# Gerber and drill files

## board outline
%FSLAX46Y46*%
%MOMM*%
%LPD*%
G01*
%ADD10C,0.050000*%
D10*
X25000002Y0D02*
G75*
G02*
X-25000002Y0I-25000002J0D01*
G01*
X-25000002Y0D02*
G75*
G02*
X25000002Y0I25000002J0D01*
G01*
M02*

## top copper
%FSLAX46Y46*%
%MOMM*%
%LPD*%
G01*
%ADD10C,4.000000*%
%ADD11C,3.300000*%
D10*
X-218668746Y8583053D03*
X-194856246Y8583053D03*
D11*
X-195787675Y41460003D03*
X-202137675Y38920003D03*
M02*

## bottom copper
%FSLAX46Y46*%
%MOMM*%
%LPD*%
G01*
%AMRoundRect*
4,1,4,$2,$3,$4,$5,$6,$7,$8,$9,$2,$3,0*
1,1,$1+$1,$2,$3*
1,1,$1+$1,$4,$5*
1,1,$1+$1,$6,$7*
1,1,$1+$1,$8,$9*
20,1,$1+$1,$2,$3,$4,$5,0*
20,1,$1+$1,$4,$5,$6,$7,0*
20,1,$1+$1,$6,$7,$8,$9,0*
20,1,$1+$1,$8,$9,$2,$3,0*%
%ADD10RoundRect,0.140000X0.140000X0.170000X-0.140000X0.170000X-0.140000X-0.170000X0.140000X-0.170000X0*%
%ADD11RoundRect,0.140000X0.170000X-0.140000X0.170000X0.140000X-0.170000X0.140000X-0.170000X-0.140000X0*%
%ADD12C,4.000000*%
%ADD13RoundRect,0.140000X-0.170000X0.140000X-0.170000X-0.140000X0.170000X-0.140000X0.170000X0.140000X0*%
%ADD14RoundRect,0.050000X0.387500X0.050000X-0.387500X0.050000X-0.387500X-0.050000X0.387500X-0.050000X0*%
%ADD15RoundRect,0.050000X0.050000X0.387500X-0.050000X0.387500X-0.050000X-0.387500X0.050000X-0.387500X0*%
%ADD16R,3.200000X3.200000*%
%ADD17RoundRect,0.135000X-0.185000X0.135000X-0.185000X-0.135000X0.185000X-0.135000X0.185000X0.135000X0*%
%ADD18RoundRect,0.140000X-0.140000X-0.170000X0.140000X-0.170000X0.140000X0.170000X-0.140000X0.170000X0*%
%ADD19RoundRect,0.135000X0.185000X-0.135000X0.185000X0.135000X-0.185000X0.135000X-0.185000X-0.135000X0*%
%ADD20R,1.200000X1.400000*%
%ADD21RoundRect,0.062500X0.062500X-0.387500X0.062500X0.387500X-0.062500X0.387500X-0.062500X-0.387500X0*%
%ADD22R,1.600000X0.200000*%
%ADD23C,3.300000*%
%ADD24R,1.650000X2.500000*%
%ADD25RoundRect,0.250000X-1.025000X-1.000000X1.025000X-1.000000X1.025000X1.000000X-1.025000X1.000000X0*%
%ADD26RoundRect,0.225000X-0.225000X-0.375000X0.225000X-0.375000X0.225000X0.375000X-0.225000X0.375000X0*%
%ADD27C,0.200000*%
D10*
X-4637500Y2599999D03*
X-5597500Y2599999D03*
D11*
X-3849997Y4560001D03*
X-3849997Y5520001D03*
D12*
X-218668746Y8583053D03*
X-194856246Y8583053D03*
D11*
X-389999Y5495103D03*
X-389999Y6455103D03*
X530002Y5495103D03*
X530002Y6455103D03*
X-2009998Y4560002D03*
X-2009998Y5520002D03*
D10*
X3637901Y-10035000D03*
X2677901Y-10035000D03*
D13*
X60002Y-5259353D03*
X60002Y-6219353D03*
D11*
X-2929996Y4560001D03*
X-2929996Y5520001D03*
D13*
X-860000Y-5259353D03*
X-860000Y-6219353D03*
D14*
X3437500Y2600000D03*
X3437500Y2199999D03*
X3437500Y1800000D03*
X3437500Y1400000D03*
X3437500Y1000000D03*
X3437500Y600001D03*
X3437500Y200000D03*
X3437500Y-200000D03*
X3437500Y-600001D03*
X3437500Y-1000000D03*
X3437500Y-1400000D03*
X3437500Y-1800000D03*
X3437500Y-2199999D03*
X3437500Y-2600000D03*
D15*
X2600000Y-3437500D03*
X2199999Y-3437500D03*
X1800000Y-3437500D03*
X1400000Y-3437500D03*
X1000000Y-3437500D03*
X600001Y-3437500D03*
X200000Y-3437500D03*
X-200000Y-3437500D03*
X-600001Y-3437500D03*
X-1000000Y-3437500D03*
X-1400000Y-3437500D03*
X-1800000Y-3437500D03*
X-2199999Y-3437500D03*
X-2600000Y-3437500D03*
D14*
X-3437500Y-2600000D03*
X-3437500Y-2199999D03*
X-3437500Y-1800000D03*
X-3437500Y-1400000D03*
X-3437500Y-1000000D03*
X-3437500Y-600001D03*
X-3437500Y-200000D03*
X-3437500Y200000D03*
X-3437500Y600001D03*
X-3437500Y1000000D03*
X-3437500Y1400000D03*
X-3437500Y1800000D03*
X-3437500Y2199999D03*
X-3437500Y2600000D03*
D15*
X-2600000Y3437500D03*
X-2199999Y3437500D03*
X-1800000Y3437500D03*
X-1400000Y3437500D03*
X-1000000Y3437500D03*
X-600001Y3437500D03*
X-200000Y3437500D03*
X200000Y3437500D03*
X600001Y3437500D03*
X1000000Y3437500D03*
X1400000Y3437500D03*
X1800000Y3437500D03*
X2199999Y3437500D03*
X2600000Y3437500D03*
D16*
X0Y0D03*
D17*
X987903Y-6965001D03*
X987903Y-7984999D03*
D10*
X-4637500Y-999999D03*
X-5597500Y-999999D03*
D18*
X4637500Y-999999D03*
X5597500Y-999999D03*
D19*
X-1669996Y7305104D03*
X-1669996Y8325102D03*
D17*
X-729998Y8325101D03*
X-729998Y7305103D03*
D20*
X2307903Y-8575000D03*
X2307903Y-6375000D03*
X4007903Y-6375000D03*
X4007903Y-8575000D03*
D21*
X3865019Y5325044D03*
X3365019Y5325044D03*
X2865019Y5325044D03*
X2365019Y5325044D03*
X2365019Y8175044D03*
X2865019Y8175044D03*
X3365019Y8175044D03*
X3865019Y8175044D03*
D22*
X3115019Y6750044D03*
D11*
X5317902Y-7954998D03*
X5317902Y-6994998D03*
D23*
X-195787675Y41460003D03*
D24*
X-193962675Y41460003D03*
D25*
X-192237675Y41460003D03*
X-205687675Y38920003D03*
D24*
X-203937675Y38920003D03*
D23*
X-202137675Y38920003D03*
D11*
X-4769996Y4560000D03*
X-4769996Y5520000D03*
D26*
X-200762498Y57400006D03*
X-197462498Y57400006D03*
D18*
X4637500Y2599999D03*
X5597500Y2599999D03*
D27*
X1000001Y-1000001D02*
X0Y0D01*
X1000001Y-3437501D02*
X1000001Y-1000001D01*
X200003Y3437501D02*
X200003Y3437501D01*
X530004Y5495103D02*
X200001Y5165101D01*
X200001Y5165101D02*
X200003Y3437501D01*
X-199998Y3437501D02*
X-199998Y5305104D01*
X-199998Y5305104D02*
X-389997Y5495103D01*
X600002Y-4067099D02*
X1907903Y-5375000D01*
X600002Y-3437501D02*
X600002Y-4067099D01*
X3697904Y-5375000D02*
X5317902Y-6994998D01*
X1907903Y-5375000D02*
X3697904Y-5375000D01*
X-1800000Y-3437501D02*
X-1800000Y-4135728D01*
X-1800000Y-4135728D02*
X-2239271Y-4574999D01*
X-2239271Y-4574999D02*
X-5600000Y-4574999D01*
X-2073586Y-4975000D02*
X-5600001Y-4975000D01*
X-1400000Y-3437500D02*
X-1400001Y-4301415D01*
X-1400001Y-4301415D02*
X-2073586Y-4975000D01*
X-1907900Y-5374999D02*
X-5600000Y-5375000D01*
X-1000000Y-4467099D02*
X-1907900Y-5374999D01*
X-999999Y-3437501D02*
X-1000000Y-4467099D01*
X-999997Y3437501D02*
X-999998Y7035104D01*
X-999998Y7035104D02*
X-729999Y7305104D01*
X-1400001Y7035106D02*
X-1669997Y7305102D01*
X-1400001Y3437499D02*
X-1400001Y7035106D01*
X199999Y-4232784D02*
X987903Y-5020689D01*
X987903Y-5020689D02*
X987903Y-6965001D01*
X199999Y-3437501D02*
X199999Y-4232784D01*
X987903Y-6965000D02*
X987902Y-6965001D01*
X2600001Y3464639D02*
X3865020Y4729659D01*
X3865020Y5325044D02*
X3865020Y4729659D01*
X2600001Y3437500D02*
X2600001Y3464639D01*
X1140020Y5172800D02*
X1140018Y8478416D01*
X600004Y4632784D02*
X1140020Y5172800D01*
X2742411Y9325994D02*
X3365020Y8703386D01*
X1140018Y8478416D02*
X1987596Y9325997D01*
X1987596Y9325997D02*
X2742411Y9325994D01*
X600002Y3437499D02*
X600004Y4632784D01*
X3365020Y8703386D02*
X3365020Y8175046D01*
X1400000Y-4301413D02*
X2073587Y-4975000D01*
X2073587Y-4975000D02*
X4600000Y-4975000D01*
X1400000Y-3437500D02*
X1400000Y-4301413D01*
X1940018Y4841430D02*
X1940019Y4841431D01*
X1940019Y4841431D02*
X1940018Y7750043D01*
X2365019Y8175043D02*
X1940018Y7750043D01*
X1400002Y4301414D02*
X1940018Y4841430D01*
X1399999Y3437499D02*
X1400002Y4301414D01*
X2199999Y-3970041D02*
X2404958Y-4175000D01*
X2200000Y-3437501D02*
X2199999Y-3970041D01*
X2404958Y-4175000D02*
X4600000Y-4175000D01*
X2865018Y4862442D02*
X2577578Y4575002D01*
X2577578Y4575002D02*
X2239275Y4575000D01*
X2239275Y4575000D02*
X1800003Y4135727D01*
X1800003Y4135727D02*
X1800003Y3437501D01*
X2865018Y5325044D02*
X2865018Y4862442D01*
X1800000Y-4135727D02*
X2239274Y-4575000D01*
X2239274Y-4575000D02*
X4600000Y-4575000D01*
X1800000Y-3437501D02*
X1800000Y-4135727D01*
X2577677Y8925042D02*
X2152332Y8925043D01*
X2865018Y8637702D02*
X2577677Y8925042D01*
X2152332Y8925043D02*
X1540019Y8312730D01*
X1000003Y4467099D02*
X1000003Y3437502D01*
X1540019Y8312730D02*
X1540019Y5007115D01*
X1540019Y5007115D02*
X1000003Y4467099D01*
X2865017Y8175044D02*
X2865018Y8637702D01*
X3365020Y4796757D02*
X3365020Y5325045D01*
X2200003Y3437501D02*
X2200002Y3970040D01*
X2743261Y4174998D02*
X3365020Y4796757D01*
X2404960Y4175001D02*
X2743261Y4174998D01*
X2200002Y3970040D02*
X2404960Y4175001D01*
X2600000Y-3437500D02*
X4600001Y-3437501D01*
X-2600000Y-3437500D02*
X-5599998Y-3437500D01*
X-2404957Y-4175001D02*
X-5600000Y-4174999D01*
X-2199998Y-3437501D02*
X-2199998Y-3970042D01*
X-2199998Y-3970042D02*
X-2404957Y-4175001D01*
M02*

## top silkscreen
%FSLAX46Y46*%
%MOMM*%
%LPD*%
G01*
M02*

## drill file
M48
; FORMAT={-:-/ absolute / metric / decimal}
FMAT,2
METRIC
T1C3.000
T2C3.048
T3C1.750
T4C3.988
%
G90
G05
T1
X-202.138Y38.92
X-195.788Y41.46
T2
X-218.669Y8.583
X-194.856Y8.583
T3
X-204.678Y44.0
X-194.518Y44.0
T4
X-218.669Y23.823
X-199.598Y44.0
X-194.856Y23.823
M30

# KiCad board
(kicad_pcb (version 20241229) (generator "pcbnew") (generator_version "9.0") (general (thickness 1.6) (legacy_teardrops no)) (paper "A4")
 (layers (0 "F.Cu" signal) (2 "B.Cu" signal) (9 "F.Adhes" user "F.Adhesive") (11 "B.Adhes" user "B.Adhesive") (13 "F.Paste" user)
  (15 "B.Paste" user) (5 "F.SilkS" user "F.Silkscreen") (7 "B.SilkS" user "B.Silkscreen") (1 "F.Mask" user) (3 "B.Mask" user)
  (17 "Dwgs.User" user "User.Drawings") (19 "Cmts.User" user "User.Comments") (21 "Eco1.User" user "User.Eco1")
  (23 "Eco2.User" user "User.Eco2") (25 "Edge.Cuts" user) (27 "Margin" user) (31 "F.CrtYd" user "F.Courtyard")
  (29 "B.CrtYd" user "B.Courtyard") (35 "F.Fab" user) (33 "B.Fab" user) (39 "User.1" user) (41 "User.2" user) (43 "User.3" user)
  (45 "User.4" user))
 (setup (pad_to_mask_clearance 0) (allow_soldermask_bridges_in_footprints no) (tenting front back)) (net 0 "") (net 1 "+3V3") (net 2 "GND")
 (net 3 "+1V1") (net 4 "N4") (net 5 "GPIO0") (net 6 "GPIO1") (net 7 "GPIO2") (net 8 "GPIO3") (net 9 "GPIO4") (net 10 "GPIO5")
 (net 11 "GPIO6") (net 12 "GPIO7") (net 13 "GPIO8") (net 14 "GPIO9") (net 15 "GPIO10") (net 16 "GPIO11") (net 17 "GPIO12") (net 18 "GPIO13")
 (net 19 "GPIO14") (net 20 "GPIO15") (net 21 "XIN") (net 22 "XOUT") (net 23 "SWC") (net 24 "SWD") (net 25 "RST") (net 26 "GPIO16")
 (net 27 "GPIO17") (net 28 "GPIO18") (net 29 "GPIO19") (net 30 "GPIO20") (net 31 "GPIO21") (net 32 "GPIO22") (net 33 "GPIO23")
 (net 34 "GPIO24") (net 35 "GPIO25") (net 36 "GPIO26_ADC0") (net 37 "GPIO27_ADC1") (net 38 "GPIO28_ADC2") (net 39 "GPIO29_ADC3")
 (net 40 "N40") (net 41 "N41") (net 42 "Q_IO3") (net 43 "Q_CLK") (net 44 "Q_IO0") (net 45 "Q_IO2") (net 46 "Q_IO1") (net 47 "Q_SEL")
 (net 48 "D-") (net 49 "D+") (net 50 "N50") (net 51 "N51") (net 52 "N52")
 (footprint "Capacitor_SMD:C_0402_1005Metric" (layer "B.Cu") (at -5.1175 -2.599999 180)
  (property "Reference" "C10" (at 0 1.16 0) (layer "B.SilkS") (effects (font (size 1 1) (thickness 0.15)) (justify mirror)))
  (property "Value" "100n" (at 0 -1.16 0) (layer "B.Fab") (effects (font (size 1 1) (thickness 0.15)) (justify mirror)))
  (pad "1" smd roundrect (at -0.48 0 180) (size 0.56 0.62) (layers "B.Cu" "B.Mask" "B.Paste") (roundrect_rratio 0.25) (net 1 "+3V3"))
  (pad "2" smd roundrect (at 0.48 0 180) (size 0.56 0.62) (layers "B.Cu" "B.Mask" "B.Paste") (roundrect_rratio 0.25) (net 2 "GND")))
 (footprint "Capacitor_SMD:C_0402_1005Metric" (layer "B.Cu") (at -3.849997 -5.040001 90)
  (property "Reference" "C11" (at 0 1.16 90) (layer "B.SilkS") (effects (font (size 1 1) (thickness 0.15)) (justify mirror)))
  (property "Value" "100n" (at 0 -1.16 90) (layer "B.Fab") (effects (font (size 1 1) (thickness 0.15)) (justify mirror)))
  (pad "1" smd roundrect (at -0.48 0 90) (size 0.56 0.62) (layers "B.Cu" "B.Mask" "B.Paste") (roundrect_rratio 0.25) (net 1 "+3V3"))
  (pad "2" smd roundrect (at 0.48 0 90) (size 0.56 0.62) (layers "B.Cu" "B.Mask" "B.Paste") (roundrect_rratio 0.25) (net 2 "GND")))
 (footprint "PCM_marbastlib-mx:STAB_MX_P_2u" (layer "B.Cu") (at -206.762496 -15.568053)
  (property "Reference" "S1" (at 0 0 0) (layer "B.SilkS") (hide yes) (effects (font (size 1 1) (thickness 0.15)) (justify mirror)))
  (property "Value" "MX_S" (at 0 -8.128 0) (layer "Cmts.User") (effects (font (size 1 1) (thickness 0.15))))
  (pad "" np_thru_hole circle (at -11.906251 -8.255) (size 3.9878 3.9878) (drill 3.9878) (layers "*.Cu" "*.Mask"))
  (pad "" thru_hole circle (at -11.90625 6.985) (size 4 4) (drill 3.048) (layers "*.Cu" "F.Mask") (remove_unused_layers no))
  (pad "" thru_hole circle (at 11.90625 6.985) (size 4 4) (drill 3.048) (layers "*.Cu" "F.Mask") (remove_unused_layers no))
  (pad "" np_thru_hole circle (at 11.906251 -8.255) (size 3.9878 3.9878) (drill 3.9878) (layers "*.Cu" "*.Mask")))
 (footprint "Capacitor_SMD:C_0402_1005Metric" (layer "B.Cu") (at -0.389999 -5.975103 90)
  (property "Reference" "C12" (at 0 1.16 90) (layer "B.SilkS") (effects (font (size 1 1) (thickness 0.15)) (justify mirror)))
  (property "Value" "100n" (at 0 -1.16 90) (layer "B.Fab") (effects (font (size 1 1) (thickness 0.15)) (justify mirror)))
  (pad "1" smd roundrect (at -0.48 0 90) (size 0.56 0.62) (layers "B.Cu" "B.Mask" "B.Paste") (roundrect_rratio 0.25) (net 1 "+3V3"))
  (pad "2" smd roundrect (at 0.48 0 90) (size 0.56 0.62) (layers "B.Cu" "B.Mask" "B.Paste") (roundrect_rratio 0.25) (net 2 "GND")))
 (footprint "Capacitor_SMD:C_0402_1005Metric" (layer "B.Cu") (at 0.530002 -5.975103 90)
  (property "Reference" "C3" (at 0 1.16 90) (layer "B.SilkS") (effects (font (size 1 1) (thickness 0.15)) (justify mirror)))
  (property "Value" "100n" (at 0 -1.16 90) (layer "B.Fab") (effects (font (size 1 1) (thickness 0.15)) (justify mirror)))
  (pad "1" smd roundrect (at -0.48 0 90) (size 0.56 0.62) (layers "B.Cu" "B.Mask" "B.Paste") (roundrect_rratio 0.25) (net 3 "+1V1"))
  (pad "2" smd roundrect (at 0.48 0 90) (size 0.56 0.62) (layers "B.Cu" "B.Mask" "B.Paste") (roundrect_rratio 0.25) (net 2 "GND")))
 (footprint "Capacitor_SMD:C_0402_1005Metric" (layer "B.Cu") (at -2.009998 -5.040002 90)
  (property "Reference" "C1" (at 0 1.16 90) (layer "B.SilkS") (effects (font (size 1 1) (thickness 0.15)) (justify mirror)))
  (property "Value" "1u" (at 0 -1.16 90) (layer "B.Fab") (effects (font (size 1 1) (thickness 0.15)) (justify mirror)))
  (pad "1" smd roundrect (at -0.48 0 90) (size 0.56 0.62) (layers "B.Cu" "B.Mask" "B.Paste") (roundrect_rratio 0.25) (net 3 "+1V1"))
  (pad "2" smd roundrect (at 0.48 0 90) (size 0.56 0.62) (layers "B.Cu" "B.Mask" "B.Paste") (roundrect_rratio 0.25) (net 2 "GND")))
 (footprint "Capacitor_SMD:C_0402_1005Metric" (layer "B.Cu") (at 3.157901 10.035 180)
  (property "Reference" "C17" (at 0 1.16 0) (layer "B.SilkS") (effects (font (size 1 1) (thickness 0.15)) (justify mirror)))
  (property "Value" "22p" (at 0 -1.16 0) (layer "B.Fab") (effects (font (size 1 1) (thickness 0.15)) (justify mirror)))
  (pad "1" smd roundrect (at -0.48 0 180) (size 0.56 0.62) (layers "B.Cu" "B.Mask" "B.Paste") (roundrect_rratio 0.25) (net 2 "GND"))
  (pad "2" smd roundrect (at 0.48 0 180) (size 0.56 0.62) (layers "B.Cu" "B.Mask" "B.Paste") (roundrect_rratio 0.25) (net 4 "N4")))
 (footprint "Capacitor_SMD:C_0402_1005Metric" (layer "B.Cu") (at 0.060002 5.739353 -90)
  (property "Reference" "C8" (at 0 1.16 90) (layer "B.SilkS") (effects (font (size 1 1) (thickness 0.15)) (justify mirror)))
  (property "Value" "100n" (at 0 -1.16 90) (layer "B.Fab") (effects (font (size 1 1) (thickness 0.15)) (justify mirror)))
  (pad "1" smd roundrect (at -0.48 0 270) (size 0.56 0.62) (layers "B.Cu" "B.Mask" "B.Paste") (roundrect_rratio 0.25) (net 1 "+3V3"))
  (pad "2" smd roundrect (at 0.48 0 270) (size 0.56 0.62) (layers "B.Cu" "B.Mask" "B.Paste") (roundrect_rratio 0.25) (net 2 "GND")))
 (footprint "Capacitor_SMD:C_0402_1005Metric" (layer "B.Cu") (at -2.929996 -5.040001 90)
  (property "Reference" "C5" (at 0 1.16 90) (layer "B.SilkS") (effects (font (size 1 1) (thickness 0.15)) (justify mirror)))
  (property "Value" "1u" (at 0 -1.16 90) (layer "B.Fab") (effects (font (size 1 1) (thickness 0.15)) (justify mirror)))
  (pad "1" smd roundrect (at -0.48 0 90) (size 0.56 0.62) (layers "B.Cu" "B.Mask" "B.Paste") (roundrect_rratio 0.25) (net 1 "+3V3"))
  (pad "2" smd roundrect (at 0.48 0 90) (size 0.56 0.62) (layers "B.Cu" "B.Mask" "B.Paste") (roundrect_rratio 0.25) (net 2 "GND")))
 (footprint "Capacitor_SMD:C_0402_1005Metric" (layer "B.Cu") (at -0.86 5.739353 -90)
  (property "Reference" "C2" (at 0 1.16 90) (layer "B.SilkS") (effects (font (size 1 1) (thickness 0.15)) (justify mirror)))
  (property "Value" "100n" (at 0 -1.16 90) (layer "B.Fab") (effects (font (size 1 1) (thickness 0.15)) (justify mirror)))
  (pad "1" smd roundrect (at -0.48 0 270) (size 0.56 0.62) (layers "B.Cu" "B.Mask" "B.Paste") (roundrect_rratio 0.25) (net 3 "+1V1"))
  (pad "2" smd roundrect (at 0.48 0 270) (size 0.56 0.62) (layers "B.Cu" "B.Mask" "B.Paste") (roundrect_rratio 0.25) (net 2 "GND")))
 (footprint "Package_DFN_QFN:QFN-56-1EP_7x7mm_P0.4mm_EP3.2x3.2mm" (layer "B.Cu") (at 0 0 180)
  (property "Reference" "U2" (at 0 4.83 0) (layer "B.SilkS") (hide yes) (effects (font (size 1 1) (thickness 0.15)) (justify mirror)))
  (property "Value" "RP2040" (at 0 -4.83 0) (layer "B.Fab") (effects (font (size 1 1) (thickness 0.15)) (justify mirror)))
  (pad "" smd roundrect (at -0.8 -0.8 180) (size 1.29 1.29) (layers "B.Paste") (roundrect_rratio 0.193798))
  (pad "" smd roundrect (at -0.8 0.8 180) (size 1.29 1.29) (layers "B.Paste") (roundrect_rratio 0.193798))
  (pad "" smd roundrect (at 0.8 -0.8 180) (size 1.29 1.29) (layers "B.Paste") (roundrect_rratio 0.193798))
  (pad "" smd roundrect (at 0.8 0.8 180) (size 1.29 1.29) (layers "B.Paste") (roundrect_rratio 0.193798))
  (pad "1" smd roundrect (at -3.4375 2.6 180) (size 0.875 0.2) (layers "B.Cu" "B.Mask" "B.Paste") (roundrect_rratio 0.25) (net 1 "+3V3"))
  (pad "2" smd roundrect (at -3.4375 2.199999 180) (size 0.875 0.2) (layers "B.Cu" "B.Mask" "B.Paste") (roundrect_rratio 0.25)
   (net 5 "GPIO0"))
  (pad "3" smd roundrect (at -3.4375 1.8 180) (size 0.875 0.2) (layers "B.Cu" "B.Mask" "B.Paste") (roundrect_rratio 0.25) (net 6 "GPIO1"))
  (pad "4" smd roundrect (at -3.4375 1.4 180) (size 0.875 0.2) (layers "B.Cu" "B.Mask" "B.Paste") (roundrect_rratio 0.25) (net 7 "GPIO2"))
  (pad "5" smd roundrect (at -3.4375 1 180) (size 0.875 0.2) (layers "B.Cu" "B.Mask" "B.Paste") (roundrect_rratio 0.25) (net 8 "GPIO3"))
  (pad "6" smd roundrect (at -3.4375 0.600001 180) (size 0.875 0.2) (layers "B.Cu" "B.Mask" "B.Paste") (roundrect_rratio 0.25)
   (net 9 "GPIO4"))
  (pad "7" smd roundrect (at -3.4375 0.2 180) (size 0.875 0.2) (layers "B.Cu" "B.Mask" "B.Paste") (roundrect_rratio 0.25) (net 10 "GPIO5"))
  (pad "8" smd roundrect (at -3.4375 -0.2 180) (size 0.875 0.2) (layers "B.Cu" "B.Mask" "B.Paste") (roundrect_rratio 0.25) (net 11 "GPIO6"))
  (pad "9" smd roundrect (at -3.4375 -0.600001 180) (size 0.875 0.2) (layers "B.Cu" "B.Mask" "B.Paste") (roundrect_rratio 0.25)
   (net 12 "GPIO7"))
  (pad "10" smd roundrect (at -3.4375 -1 180) (size 0.875 0.2) (layers "B.Cu" "B.Mask" "B.Paste") (roundrect_rratio 0.25) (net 1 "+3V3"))
  (pad "11" smd roundrect (at -3.4375 -1.4 180) (size 0.875 0.2) (layers "B.Cu" "B.Mask" "B.Paste") (roundrect_rratio 0.25) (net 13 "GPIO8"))
  (pad "12" smd roundrect (at -3.4375 -1.8 180) (size 0.875 0.2) (layers "B.Cu" "B.Mask" "B.Paste") (roundrect_rratio 0.25) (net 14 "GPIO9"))
  (pad "13" smd roundrect (at -3.4375 -2.199999 180) (size 0.875 0.2) (layers "B.Cu" "B.Mask" "B.Paste") (roundrect_rratio 0.25)
   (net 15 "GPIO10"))
  (pad "14" smd roundrect (at -3.4375 -2.6 180) (size 0.875 0.2) (layers "B.Cu" "B.Mask" "B.Paste") (roundrect_rratio 0.25)
   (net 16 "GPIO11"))
  (pad "15" smd roundrect (at -2.6 -3.4375 180) (size 0.2 0.875) (layers "B.Cu" "B.Mask" "B.Paste") (roundrect_rratio 0.25)
   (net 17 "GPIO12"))
  (pad "16" smd roundrect (at -2.199999 -3.4375 180) (size 0.2 0.875) (layers "B.Cu" "B.Mask" "B.Paste") (roundrect_rratio 0.25)
   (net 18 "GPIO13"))
  (pad "17" smd roundrect (at -1.8 -3.4375 180) (size 0.2 0.875) (layers "B.Cu" "B.Mask" "B.Paste") (roundrect_rratio 0.25)
   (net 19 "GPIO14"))
  (pad "18" smd roundrect (at -1.4 -3.4375 180) (size 0.2 0.875) (layers "B.Cu" "B.Mask" "B.Paste") (roundrect_rratio 0.25)
   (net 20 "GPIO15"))
  (pad "19" smd roundrect (at -1 -3.4375 180) (size 0.2 0.875) (layers "B.Cu" "B.Mask" "B.Paste") (roundrect_rratio 0.25) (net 2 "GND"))
  (pad "20" smd roundrect (at -0.600001 -3.4375 180) (size 0.2 0.875) (layers "B.Cu" "B.Mask" "B.Paste") (roundrect_rratio 0.25)
   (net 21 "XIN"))
  (pad "21" smd roundrect (at -0.2 -3.4375 180) (size 0.2 0.875) (layers "B.Cu" "B.Mask" "B.Paste") (roundrect_rratio 0.25) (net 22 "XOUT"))
  (pad "22" smd roundrect (at 0.2 -3.4375 180) (size 0.2 0.875) (layers "B.Cu" "B.Mask" "B.Paste") (roundrect_rratio 0.25) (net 1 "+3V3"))
  (pad "23" smd roundrect (at 0.600001 -3.4375 180) (size 0.2 0.875) (layers "B.Cu" "B.Mask" "B.Paste") (roundrect_rratio 0.25)
   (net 3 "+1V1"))
  (pad "24" smd roundrect (at 1 -3.4375 180) (size 0.2 0.875) (layers "B.Cu" "B.Mask" "B.Paste") (roundrect_rratio 0.25) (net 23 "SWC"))
  (pad "25" smd roundrect (at 1.4 -3.4375 180) (size 0.2 0.875) (layers "B.Cu" "B.Mask" "B.Paste") (roundrect_rratio 0.25) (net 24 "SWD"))
  (pad "26" smd roundrect (at 1.8 -3.4375 180) (size 0.2 0.875) (layers "B.Cu" "B.Mask" "B.Paste") (roundrect_rratio 0.25) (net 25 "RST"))
  (pad "27" smd roundrect (at 2.199999 -3.4375 180) (size 0.2 0.875) (layers "B.Cu" "B.Mask" "B.Paste") (roundrect_rratio 0.25)
   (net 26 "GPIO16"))
  (pad "28" smd roundrect (at 2.6 -3.4375 180) (size 0.2 0.875) (layers "B.Cu" "B.Mask" "B.Paste") (roundrect_rratio 0.25) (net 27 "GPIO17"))
  (pad "29" smd roundrect (at 3.4375 -2.6 180) (size 0.875 0.2) (layers "B.Cu" "B.Mask" "B.Paste") (roundrect_rratio 0.25) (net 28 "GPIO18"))
  (pad "30" smd roundrect (at 3.4375 -2.199999 180) (size 0.875 0.2) (layers "B.Cu" "B.Mask" "B.Paste") (roundrect_rratio 0.25)
   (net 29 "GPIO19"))
  (pad "31" smd roundrect (at 3.4375 -1.8 180) (size 0.875 0.2) (layers "B.Cu" "B.Mask" "B.Paste") (roundrect_rratio 0.25) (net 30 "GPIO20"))
  (pad "32" smd roundrect (at 3.4375 -1.4 180) (size 0.875 0.2) (layers "B.Cu" "B.Mask" "B.Paste") (roundrect_rratio 0.25) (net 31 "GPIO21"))
  (pad "33" smd roundrect (at 3.4375 -1 180) (size 0.875 0.2) (layers "B.Cu" "B.Mask" "B.Paste") (roundrect_rratio 0.25) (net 1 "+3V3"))
  (pad "34" smd roundrect (at 3.4375 -0.600001 180) (size 0.875 0.2) (layers "B.Cu" "B.Mask" "B.Paste") (roundrect_rratio 0.25)
   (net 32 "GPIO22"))
  (pad "35" smd roundrect (at 3.4375 -0.2 180) (size 0.875 0.2) (layers "B.Cu" "B.Mask" "B.Paste") (roundrect_rratio 0.25) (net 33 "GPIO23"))
  (pad "36" smd roundrect (at 3.4375 0.2 180) (size 0.875 0.2) (layers "B.Cu" "B.Mask" "B.Paste") (roundrect_rratio 0.25) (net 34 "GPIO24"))
  (pad "37" smd roundrect (at 3.4375 0.600001 180) (size 0.875 0.2) (layers "B.Cu" "B.Mask" "B.Paste") (roundrect_rratio 0.25)
   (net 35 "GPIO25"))
  (pad "38" smd roundrect (at 3.4375 1 180) (size 0.875 0.2) (layers "B.Cu" "B.Mask" "B.Paste") (roundrect_rratio 0.25)
   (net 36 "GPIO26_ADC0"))
  (pad "39" smd roundrect (at 3.4375 1.4 180) (size 0.875 0.2) (layers "B.Cu" "B.Mask" "B.Paste") (roundrect_rratio 0.25)
   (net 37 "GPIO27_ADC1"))
  (pad "40" smd roundrect (at 3.4375 1.8 180) (size 0.875 0.2) (layers "B.Cu" "B.Mask" "B.Paste") (roundrect_rratio 0.25)
   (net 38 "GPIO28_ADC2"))
  (pad "41" smd roundrect (at 3.4375 2.199999 180) (size 0.875 0.2) (layers "B.Cu" "B.Mask" "B.Paste") (roundrect_rratio 0.25)
   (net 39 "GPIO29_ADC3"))
  (pad "42" smd roundrect (at 3.4375 2.6 180) (size 0.875 0.2) (layers "B.Cu" "B.Mask" "B.Paste") (roundrect_rratio 0.25) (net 1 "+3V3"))
  (pad "43" smd roundrect (at 2.6 3.4375 180) (size 0.2 0.875) (layers "B.Cu" "B.Mask" "B.Paste") (roundrect_rratio 0.25) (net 1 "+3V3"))
  (pad "44" smd roundrect (at 2.199999 3.4375 180) (size 0.2 0.875) (layers "B.Cu" "B.Mask" "B.Paste") (roundrect_rratio 0.25)
   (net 1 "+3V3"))
  (pad "45" smd roundrect (at 1.8 3.4375 180) (size 0.2 0.875) (layers "B.Cu" "B.Mask" "B.Paste") (roundrect_rratio 0.25) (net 3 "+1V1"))
  (pad "46" smd roundrect (at 1.4 3.4375 180) (size 0.2 0.875) (layers "B.Cu" "B.Mask" "B.Paste") (roundrect_rratio 0.25) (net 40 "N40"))
  (pad "47" smd roundrect (at 1 3.4375 180) (size 0.2 0.875) (layers "B.Cu" "B.Mask" "B.Paste") (roundrect_rratio 0.25) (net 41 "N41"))
  (pad "48" smd roundrect (at 0.600001 3.4375 180) (size 0.2 0.875) (layers "B.Cu" "B.Mask" "B.Paste") (roundrect_rratio 0.25)
   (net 1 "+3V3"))
  (pad "49" smd roundrect (at 0.2 3.4375 180) (size 0.2 0.875) (layers "B.Cu" "B.Mask" "B.Paste") (roundrect_rratio 0.25) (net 1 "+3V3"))
  (pad "50" smd roundrect (at -0.2 3.4375 180) (size 0.2 0.875) (layers "B.Cu" "B.Mask" "B.Paste") (roundrect_rratio 0.25) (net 3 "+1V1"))
  (pad "51" smd roundrect (at -0.600001 3.4375 180) (size 0.2 0.875) (layers "B.Cu" "B.Mask" "B.Paste") (roundrect_rratio 0.25)
   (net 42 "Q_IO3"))
  (pad "52" smd roundrect (at -1 3.4375 180) (size 0.2 0.875) (layers "B.Cu" "B.Mask" "B.Paste") (roundrect_rratio 0.25) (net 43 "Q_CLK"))
  (pad "53" smd roundrect (at -1.4 3.4375 180) (size 0.2 0.875) (layers "B.Cu" "B.Mask" "B.Paste") (roundrect_rratio 0.25) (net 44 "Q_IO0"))
  (pad "54" smd roundrect (at -1.8 3.4375 180) (size 0.2 0.875) (layers "B.Cu" "B.Mask" "B.Paste") (roundrect_rratio 0.25) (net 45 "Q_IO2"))
  (pad "55" smd roundrect (at -2.199999 3.4375 180) (size 0.2 0.875) (layers "B.Cu" "B.Mask" "B.Paste") (roundrect_rratio 0.25)
   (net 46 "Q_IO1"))
  (pad "56" smd roundrect (at -2.6 3.4375 180) (size 0.2 0.875) (layers "B.Cu" "B.Mask" "B.Paste") (roundrect_rratio 0.25) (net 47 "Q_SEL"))
  (pad "57" smd rect (at 0 0 180) (size 3.2 3.2) (layers "B.Cu" "B.Mask") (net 2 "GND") (zone_connect 2)))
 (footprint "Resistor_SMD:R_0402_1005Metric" (layer "B.Cu") (at 0.987903 7.475 -90)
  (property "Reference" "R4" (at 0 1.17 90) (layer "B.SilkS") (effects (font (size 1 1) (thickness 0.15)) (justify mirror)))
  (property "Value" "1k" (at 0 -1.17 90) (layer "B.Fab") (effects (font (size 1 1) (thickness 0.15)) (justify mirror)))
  (pad "1" smd roundrect (at -0.509999 0 270) (size 0.54 0.64) (layers "B.Cu" "B.Mask" "B.Paste") (roundrect_rratio 0.25) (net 22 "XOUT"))
  (pad "2" smd roundrect (at 0.509999 0 270) (size 0.54 0.64) (layers "B.Cu" "B.Mask" "B.Paste") (roundrect_rratio 0.25) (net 4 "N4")))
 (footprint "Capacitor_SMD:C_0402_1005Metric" (layer "B.Cu") (at -5.1175 0.999999 180)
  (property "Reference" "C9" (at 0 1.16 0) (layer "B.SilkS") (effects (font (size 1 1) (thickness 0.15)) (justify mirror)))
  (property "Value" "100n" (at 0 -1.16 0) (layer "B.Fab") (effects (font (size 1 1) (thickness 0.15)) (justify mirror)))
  (pad "1" smd roundrect (at -0.48 0 180) (size 0.56 0.62) (layers "B.Cu" "B.Mask" "B.Paste") (roundrect_rratio 0.25) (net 1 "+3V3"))
  (pad "2" smd roundrect (at 0.48 0 180) (size 0.56 0.62) (layers "B.Cu" "B.Mask" "B.Paste") (roundrect_rratio 0.25) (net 2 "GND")))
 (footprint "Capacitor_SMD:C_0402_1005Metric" (layer "B.Cu") (at 5.1175 0.999999)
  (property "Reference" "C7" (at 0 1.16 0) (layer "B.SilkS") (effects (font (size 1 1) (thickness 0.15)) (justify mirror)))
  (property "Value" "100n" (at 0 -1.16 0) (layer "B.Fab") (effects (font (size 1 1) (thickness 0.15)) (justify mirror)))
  (pad "1" smd roundrect (at -0.48 0) (size 0.56 0.62) (layers "B.Cu" "B.Mask" "B.Paste") (roundrect_rratio 0.25) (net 1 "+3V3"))
  (pad "2" smd roundrect (at 0.48 0) (size 0.56 0.62) (layers "B.Cu" "B.Mask" "B.Paste") (roundrect_rratio 0.25) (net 2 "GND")))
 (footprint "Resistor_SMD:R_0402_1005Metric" (layer "B.Cu") (at -1.669996 -7.815103 90)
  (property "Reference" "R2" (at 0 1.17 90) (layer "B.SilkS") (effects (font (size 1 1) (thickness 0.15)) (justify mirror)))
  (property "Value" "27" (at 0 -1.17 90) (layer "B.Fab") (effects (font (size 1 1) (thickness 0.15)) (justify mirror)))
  (pad "1" smd roundrect (at -0.509999 0 90) (size 0.54 0.64) (layers "B.Cu" "B.Mask" "B.Paste") (roundrect_rratio 0.25) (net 40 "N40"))
  (pad "2" smd roundrect (at 0.509999 0 90) (size 0.54 0.64) (layers "B.Cu" "B.Mask" "B.Paste") (roundrect_rratio 0.25) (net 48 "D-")))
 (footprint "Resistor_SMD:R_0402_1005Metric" (layer "B.Cu") (at -0.729998 -7.815102 -90)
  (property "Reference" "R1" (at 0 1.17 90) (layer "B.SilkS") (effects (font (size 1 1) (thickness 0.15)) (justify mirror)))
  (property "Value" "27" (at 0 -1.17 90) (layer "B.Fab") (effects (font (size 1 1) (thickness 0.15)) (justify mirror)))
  (pad "1" smd roundrect (at -0.509999 0 270) (size 0.54 0.64) (layers "B.Cu" "B.Mask" "B.Paste") (roundrect_rratio 0.25) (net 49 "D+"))
  (pad "2" smd roundrect (at 0.509999 0 270) (size 0.54 0.64) (layers "B.Cu" "B.Mask" "B.Paste") (roundrect_rratio 0.25) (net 41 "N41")))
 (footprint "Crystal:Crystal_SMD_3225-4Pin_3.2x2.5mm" (layer "B.Cu") (at 3.157903 7.475 90)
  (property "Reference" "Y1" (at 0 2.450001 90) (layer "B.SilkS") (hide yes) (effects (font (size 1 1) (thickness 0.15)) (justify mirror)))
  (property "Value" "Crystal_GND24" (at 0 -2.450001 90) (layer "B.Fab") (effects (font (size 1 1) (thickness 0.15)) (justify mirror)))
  (pad "1" smd rect (at -1.1 -0.85 90) (size 1.4 1.2) (layers "B.Cu" "B.Mask" "B.Paste") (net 4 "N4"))
  (pad "2" smd rect (at 1.1 -0.85 90) (size 1.4 1.2) (layers "B.Cu" "B.Mask" "B.Paste") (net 2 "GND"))
  (pad "3" smd rect (at 1.1 0.85 90) (size 1.4 1.2) (layers "B.Cu" "B.Mask" "B.Paste") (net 21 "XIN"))
  (pad "4" smd rect (at -1.1 0.85 90) (size 1.4 1.2) (layers "B.Cu" "B.Mask" "B.Paste") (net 2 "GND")))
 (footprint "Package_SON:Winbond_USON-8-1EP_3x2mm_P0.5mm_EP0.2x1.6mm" (layer "B.Cu") (at 3.115019 -6.750044 90)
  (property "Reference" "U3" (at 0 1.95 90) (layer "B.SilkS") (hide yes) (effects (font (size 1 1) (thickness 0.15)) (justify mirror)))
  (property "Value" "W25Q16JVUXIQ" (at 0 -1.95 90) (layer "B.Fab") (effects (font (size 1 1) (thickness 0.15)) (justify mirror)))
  (pad "" smd roundrect (at 0 0 90) (size 0.16 1.29) (layers "B.Paste") (roundrect_rratio 0.25))
  (pad "1" smd roundrect (at -1.425 0.75 90) (size 0.9 0.25) (layers "B.Cu" "B.Mask" "B.Paste") (roundrect_rratio 0.25) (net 47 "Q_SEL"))
  (pad "2" smd roundrect (at -1.425 0.25 90) (size 0.9 0.25) (layers "B.Cu" "B.Mask" "B.Paste") (roundrect_rratio 0.25) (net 46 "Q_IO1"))
  (pad "3" smd roundrect (at -1.425 -0.25 90) (size 0.9 0.25) (layers "B.Cu" "B.Mask" "B.Paste") (roundrect_rratio 0.25) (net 45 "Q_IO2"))
  (pad "4" smd roundrect (at -1.425 -0.75 90) (size 0.9 0.25) (layers "B.Cu" "B.Mask" "B.Paste") (roundrect_rratio 0.25) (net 2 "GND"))
  (pad "5" smd roundrect (at 1.425 -0.75 90) (size 0.9 0.25) (layers "B.Cu" "B.Mask" "B.Paste") (roundrect_rratio 0.25) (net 44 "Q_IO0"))
  (pad "6" smd roundrect (at 1.425 -0.25 90) (size 0.9 0.25) (layers "B.Cu" "B.Mask" "B.Paste") (roundrect_rratio 0.25) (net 43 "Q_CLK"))
  (pad "7" smd roundrect (at 1.425 0.25 90) (size 0.9 0.25) (layers "B.Cu" "B.Mask" "B.Paste") (roundrect_rratio 0.25) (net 42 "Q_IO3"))
  (pad "8" smd roundrect (at 1.425 0.75 90) (size 0.9 0.25) (layers "B.Cu" "B.Mask" "B.Paste") (roundrect_rratio 0.25) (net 1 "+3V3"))
  (pad "9" smd rect (at 0 0 90) (size 0.2 1.6) (layers "B.Cu" "B.Mask") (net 2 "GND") (zone_connect 2)))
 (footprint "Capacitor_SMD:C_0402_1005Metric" (layer "B.Cu") (at 5.317902 7.474998 90)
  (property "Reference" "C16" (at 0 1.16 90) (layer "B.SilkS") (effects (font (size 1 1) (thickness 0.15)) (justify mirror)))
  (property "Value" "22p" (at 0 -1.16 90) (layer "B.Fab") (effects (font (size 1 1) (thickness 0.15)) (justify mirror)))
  (pad "1" smd roundrect (at -0.48 0 90) (size 0.56 0.62) (layers "B.Cu" "B.Mask" "B.Paste") (roundrect_rratio 0.25) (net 2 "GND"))
  (pad "2" smd roundrect (at 0.48 0 90) (size 0.56 0.62) (layers "B.Cu" "B.Mask" "B.Paste") (roundrect_rratio 0.25) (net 21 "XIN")))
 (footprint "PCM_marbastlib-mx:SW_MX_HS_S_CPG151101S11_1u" (layer "B.Cu") (at -199.597675 -44.000003)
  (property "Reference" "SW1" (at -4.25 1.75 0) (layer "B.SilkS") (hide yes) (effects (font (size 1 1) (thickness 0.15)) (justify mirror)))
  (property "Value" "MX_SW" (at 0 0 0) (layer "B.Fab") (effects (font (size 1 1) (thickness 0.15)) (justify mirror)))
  (pad "" np_thru_hole circle (at -5.079999 0) (size 1.75 1.75) (drill 1.75) (layers "*.Cu" "*.Mask"))
  (pad "" np_thru_hole circle (at 0 0) (size 3.9878 3.9878) (drill 3.9878) (layers "*.Cu" "*.Mask"))
  (pad "" np_thru_hole circle (at 5.079999 0) (size 1.75 1.75) (drill 1.75) (layers "*.Cu" "*.Mask"))
  (pad "1" thru_hole circle (at 3.81 2.54) (size 3.3 3.3) (drill 3) (layers "*.Cu" "*.Mask") (remove_unused_layers no) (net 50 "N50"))
  (pad "1" smd rect (at 5.635 2.54 180) (size 1.65 2.5) (layers "B.Cu") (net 50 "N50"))
  (pad "1" smd roundrect (at 7.36 2.54) (size 2.55 2.5) (layers "B.Cu" "B.Mask" "B.Paste") (roundrect_rratio 0.1) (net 50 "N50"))
  (pad "2" smd roundrect (at -6.09 5.08) (size 2.55 2.5) (layers "B.Cu" "B.Mask" "B.Paste") (roundrect_rratio 0.1) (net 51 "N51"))
  (pad "2" smd rect (at -4.34 5.08) (size 1.65 2.5) (layers "B.Cu") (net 51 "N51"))
  (pad "2" thru_hole circle (at -2.54 5.08) (size 3.3 3.3) (drill 3) (layers "*.Cu" "*.Mask") (remove_unused_layers no) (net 51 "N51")))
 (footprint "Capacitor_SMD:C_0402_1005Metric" (layer "B.Cu") (at -4.769996 -5.04 90)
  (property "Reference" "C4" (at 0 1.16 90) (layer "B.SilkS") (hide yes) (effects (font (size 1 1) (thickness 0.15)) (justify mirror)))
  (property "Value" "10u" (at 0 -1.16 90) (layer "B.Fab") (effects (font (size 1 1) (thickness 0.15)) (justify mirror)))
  (pad "1" smd roundrect (at -0.48 0 90) (size 0.56 0.62) (layers "B.Cu" "B.Mask" "B.Paste") (roundrect_rratio 0.25) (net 1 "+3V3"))
  (pad "2" smd roundrect (at 0.48 0 90) (size 0.56 0.62) (layers "B.Cu" "B.Mask" "B.Paste") (roundrect_rratio 0.25) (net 2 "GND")))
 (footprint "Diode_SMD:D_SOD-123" (layer "B.Cu") (at -199.112498 -57.400006)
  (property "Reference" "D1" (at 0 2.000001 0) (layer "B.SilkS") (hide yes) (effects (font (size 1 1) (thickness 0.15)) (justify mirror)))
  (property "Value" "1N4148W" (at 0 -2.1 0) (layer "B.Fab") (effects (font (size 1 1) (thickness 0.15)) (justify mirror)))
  (pad "1" smd roundrect (at -1.65 0) (size 0.9 1.2) (layers "B.Cu" "B.Mask" "B.Paste") (roundrect_rratio 0.25) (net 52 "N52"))
  (pad "2" smd roundrect (at 1.65 0) (size 0.9 1.2) (layers "B.Cu" "B.Mask" "B.Paste") (roundrect_rratio 0.25) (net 50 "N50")))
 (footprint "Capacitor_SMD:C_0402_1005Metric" (layer "B.Cu") (at 5.1175 -2.599999)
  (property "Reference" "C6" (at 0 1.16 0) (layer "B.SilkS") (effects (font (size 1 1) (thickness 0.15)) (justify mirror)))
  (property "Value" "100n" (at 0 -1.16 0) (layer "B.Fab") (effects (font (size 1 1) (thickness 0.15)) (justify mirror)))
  (pad "1" smd roundrect (at -0.48 0) (size 0.56 0.62) (layers "B.Cu" "B.Mask" "B.Paste") (roundrect_rratio 0.25) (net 1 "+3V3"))
  (pad "2" smd roundrect (at 0.48 0) (size 0.56 0.62) (layers "B.Cu" "B.Mask" "B.Paste") (roundrect_rratio 0.25) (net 2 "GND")))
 (gr_circle (center 0 0) (end 25.000002 0) (stroke (width 0.05) (type solid)) (fill no) (layer "Edge.Cuts"))
 (segment (start 1.000001 1.000001) (end 0 0) (width 0.2) (layer "B.Cu") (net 2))
 (segment (start 1.000001 3.437501) (end 1.000001 1.000001) (width 0.2) (layer "B.Cu") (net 2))
 (segment (start 0.200003 -3.437501) (end 0.200003 -3.437501) (width 0.2) (layer "B.Cu") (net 3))
 (segment (start 0.530004 -5.495103) (end 0.200001 -5.165101) (width 0.2) (layer "B.Cu") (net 3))
 (segment (start 0.200001 -5.165101) (end 0.200003 -3.437501) (width 0.2) (layer "B.Cu") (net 3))
 (segment (start -0.199998 -3.437501) (end -0.199998 -5.305104) (width 0.2) (layer "B.Cu") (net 1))
 (segment (start -0.199998 -5.305104) (end -0.389997 -5.495103) (width 0.2) (layer "B.Cu") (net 1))
 (segment (start 0.600002 4.067099) (end 1.907903 5.375) (width 0.2) (layer "B.Cu") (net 21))
 (segment (start 0.600002 3.437501) (end 0.600002 4.067099) (width 0.2) (layer "B.Cu") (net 21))
 (segment (start 3.697904 5.375) (end 5.317902 6.994998) (width 0.2) (layer "B.Cu") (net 21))
 (segment (start 1.907903 5.375) (end 3.697904 5.375) (width 0.2) (layer "B.Cu") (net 21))
 (segment (start -1.8 3.437501) (end -1.8 4.135728) (width 0.2) (layer "B.Cu") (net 25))
 (segment (start -1.8 4.135728) (end -2.239271 4.574999) (width 0.2) (layer "B.Cu") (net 25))
 (segment (start -2.239271 4.574999) (end -5.6 4.574999) (width 0.2) (layer "B.Cu") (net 25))
 (segment (start -2.073586 4.975) (end -5.600001 4.975) (width 0.2) (layer "B.Cu") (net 24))
 (segment (start -1.4 3.4375) (end -1.400001 4.301415) (width 0.2) (layer "B.Cu") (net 24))
 (segment (start -1.400001 4.301415) (end -2.073586 4.975) (width 0.2) (layer "B.Cu") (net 24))
 (segment (start -1.9079 5.374999) (end -5.6 5.375) (width 0.2) (layer "B.Cu") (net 23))
 (segment (start -1 4.467099) (end -1.9079 5.374999) (width 0.2) (layer "B.Cu") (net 23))
 (segment (start -0.999999 3.437501) (end -1 4.467099) (width 0.2) (layer "B.Cu") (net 23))
 (segment (start -0.999997 -3.437501) (end -0.999998 -7.035104) (width 0.2) (layer "B.Cu") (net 41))
 (segment (start -0.999998 -7.035104) (end -0.729999 -7.305104) (width 0.2) (layer "B.Cu") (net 41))
 (segment (start -1.400001 -7.035106) (end -1.669997 -7.305102) (width 0.2) (layer "B.Cu") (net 40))
 (segment (start -1.400001 -3.437499) (end -1.400001 -7.035106) (width 0.2) (layer "B.Cu") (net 40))
 (segment (start 0.199999 4.232784) (end 0.987903 5.020689) (width 0.2) (layer "B.Cu") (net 22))
 (segment (start 0.987903 5.020689) (end 0.987903 6.965001) (width 0.2) (layer "B.Cu") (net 22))
 (segment (start 0.199999 3.437501) (end 0.199999 4.232784) (width 0.2) (layer "B.Cu") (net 22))
 (segment (start 0.987903 6.965) (end 0.987902 6.965001) (width 0.2) (layer "B.Cu") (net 22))
 (segment (start 2.600001 -3.464639) (end 3.86502 -4.729659) (width 0.2) (layer "B.Cu") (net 47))
 (segment (start 3.86502 -5.325044) (end 3.86502 -4.729659) (width 0.2) (layer "B.Cu") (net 47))
 (segment (start 2.600001 -3.4375) (end 2.600001 -3.464639) (width 0.2) (layer "B.Cu") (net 47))
 (segment (start 1.14002 -5.1728) (end 1.140018 -8.478416) (width 0.2) (layer "B.Cu") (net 42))
 (segment (start 0.600004 -4.632784) (end 1.14002 -5.1728) (width 0.2) (layer "B.Cu") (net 42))
 (segment (start 2.742411 -9.325994) (end 3.36502 -8.703386) (width 0.2) (layer "B.Cu") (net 42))
 (segment (start 1.140018 -8.478416) (end 1.987596 -9.325997) (width 0.2) (layer "B.Cu") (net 42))
 (segment (start 1.987596 -9.325997) (end 2.742411 -9.325994) (width 0.2) (layer "B.Cu") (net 42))
 (segment (start 0.600002 -3.437499) (end 0.600004 -4.632784) (width 0.2) (layer "B.Cu") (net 42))
 (segment (start 3.36502 -8.703386) (end 3.36502 -8.175046) (width 0.2) (layer "B.Cu") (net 42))
 (segment (start 1.4 4.301413) (end 2.073587 4.975) (width 0.2) (layer "B.Cu") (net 20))
 (segment (start 2.073587 4.975) (end 4.6 4.975) (width 0.2) (layer "B.Cu") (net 20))
 (segment (start 1.4 3.4375) (end 1.4 4.301413) (width 0.2) (layer "B.Cu") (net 20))
 (segment (start 1.940018 -4.84143) (end 1.940019 -4.841431) (width 0.2) (layer "B.Cu") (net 44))
 (segment (start 1.940019 -4.841431) (end 1.940018 -7.750043) (width 0.2) (layer "B.Cu") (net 44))
 (segment (start 2.365019 -8.175043) (end 1.940018 -7.750043) (width 0.2) (layer "B.Cu") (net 44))
 (segment (start 1.400002 -4.301414) (end 1.940018 -4.84143) (width 0.2) (layer "B.Cu") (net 44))
 (segment (start 1.399999 -3.437499) (end 1.400002 -4.301414) (width 0.2) (layer "B.Cu") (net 44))
 (segment (start 2.199999 3.970041) (end 2.404958 4.175) (width 0.2) (layer "B.Cu") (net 18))
 (segment (start 2.2 3.437501) (end 2.199999 3.970041) (width 0.2) (layer "B.Cu") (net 18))
 (segment (start 2.404958 4.175) (end 4.6 4.175) (width 0.2) (layer "B.Cu") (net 18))
 (segment (start 2.865018 -4.862442) (end 2.577578 -4.575002) (width 0.2) (layer "B.Cu") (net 45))
 (segment (start 2.577578 -4.575002) (end 2.239275 -4.575) (width 0.2) (layer "B.Cu") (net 45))
 (segment (start 2.239275 -4.575) (end 1.800003 -4.135727) (width 0.2) (layer "B.Cu") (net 45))
 (segment (start 1.800003 -4.135727) (end 1.800003 -3.437501) (width 0.2) (layer "B.Cu") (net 45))
 (segment (start 2.865018 -5.325044) (end 2.865018 -4.862442) (width 0.2) (layer "B.Cu") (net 45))
 (segment (start 1.8 4.135727) (end 2.239274 4.575) (width 0.2) (layer "B.Cu") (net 19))
 (segment (start 2.239274 4.575) (end 4.6 4.575) (width 0.2) (layer "B.Cu") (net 19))
 (segment (start 1.8 3.437501) (end 1.8 4.135727) (width 0.2) (layer "B.Cu") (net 19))
 (segment (start 2.577677 -8.925042) (end 2.152332 -8.925043) (width 0.2) (layer "B.Cu") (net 43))
 (segment (start 2.865018 -8.637702) (end 2.577677 -8.925042) (width 0.2) (layer "B.Cu") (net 43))
 (segment (start 2.152332 -8.925043) (end 1.540019 -8.31273) (width 0.2) (layer "B.Cu") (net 43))
 (segment (start 1.000003 -4.467099) (end 1.000003 -3.437502) (width 0.2) (layer "B.Cu") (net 43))
 (segment (start 1.540019 -8.31273) (end 1.540019 -5.007115) (width 0.2) (layer "B.Cu") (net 43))
 (segment (start 1.540019 -5.007115) (end 1.000003 -4.467099) (width 0.2) (layer "B.Cu") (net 43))
 (segment (start 2.865017 -8.175044) (end 2.865018 -8.637702) (width 0.2) (layer "B.Cu") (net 43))
 (segment (start 3.36502 -4.796757) (end 3.36502 -5.325045) (width 0.2) (layer "B.Cu") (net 46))
 (segment (start 2.200003 -3.437501) (end 2.200002 -3.97004) (width 0.2) (layer "B.Cu") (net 46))
 (segment (start 2.743261 -4.174998) (end 3.36502 -4.796757) (width 0.2) (layer "B.Cu") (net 46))
 (segment (start 2.40496 -4.175001) (end 2.743261 -4.174998) (width 0.2) (layer "B.Cu") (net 46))
 (segment (start 2.200002 -3.97004) (end 2.40496 -4.175001) (width 0.2) (layer "B.Cu") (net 46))
 (segment (start 2.6 3.4375) (end 4.600001 3.437501) (width 0.2) (layer "B.Cu") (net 17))
 (segment (start -2.6 3.4375) (end -5.599998 3.4375) (width 0.2) (layer "B.Cu") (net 27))
 (segment (start -2.404957 4.175001) (end -5.6 4.174999) (width 0.2) (layer "B.Cu") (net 26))
 (segment (start -2.199998 3.437501) (end -2.199998 3.970042) (width 0.2) (layer "B.Cu") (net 26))
 (segment (start -2.199998 3.970042) (end -2.404957 4.175001) (width 0.2) (layer "B.Cu") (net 26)))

